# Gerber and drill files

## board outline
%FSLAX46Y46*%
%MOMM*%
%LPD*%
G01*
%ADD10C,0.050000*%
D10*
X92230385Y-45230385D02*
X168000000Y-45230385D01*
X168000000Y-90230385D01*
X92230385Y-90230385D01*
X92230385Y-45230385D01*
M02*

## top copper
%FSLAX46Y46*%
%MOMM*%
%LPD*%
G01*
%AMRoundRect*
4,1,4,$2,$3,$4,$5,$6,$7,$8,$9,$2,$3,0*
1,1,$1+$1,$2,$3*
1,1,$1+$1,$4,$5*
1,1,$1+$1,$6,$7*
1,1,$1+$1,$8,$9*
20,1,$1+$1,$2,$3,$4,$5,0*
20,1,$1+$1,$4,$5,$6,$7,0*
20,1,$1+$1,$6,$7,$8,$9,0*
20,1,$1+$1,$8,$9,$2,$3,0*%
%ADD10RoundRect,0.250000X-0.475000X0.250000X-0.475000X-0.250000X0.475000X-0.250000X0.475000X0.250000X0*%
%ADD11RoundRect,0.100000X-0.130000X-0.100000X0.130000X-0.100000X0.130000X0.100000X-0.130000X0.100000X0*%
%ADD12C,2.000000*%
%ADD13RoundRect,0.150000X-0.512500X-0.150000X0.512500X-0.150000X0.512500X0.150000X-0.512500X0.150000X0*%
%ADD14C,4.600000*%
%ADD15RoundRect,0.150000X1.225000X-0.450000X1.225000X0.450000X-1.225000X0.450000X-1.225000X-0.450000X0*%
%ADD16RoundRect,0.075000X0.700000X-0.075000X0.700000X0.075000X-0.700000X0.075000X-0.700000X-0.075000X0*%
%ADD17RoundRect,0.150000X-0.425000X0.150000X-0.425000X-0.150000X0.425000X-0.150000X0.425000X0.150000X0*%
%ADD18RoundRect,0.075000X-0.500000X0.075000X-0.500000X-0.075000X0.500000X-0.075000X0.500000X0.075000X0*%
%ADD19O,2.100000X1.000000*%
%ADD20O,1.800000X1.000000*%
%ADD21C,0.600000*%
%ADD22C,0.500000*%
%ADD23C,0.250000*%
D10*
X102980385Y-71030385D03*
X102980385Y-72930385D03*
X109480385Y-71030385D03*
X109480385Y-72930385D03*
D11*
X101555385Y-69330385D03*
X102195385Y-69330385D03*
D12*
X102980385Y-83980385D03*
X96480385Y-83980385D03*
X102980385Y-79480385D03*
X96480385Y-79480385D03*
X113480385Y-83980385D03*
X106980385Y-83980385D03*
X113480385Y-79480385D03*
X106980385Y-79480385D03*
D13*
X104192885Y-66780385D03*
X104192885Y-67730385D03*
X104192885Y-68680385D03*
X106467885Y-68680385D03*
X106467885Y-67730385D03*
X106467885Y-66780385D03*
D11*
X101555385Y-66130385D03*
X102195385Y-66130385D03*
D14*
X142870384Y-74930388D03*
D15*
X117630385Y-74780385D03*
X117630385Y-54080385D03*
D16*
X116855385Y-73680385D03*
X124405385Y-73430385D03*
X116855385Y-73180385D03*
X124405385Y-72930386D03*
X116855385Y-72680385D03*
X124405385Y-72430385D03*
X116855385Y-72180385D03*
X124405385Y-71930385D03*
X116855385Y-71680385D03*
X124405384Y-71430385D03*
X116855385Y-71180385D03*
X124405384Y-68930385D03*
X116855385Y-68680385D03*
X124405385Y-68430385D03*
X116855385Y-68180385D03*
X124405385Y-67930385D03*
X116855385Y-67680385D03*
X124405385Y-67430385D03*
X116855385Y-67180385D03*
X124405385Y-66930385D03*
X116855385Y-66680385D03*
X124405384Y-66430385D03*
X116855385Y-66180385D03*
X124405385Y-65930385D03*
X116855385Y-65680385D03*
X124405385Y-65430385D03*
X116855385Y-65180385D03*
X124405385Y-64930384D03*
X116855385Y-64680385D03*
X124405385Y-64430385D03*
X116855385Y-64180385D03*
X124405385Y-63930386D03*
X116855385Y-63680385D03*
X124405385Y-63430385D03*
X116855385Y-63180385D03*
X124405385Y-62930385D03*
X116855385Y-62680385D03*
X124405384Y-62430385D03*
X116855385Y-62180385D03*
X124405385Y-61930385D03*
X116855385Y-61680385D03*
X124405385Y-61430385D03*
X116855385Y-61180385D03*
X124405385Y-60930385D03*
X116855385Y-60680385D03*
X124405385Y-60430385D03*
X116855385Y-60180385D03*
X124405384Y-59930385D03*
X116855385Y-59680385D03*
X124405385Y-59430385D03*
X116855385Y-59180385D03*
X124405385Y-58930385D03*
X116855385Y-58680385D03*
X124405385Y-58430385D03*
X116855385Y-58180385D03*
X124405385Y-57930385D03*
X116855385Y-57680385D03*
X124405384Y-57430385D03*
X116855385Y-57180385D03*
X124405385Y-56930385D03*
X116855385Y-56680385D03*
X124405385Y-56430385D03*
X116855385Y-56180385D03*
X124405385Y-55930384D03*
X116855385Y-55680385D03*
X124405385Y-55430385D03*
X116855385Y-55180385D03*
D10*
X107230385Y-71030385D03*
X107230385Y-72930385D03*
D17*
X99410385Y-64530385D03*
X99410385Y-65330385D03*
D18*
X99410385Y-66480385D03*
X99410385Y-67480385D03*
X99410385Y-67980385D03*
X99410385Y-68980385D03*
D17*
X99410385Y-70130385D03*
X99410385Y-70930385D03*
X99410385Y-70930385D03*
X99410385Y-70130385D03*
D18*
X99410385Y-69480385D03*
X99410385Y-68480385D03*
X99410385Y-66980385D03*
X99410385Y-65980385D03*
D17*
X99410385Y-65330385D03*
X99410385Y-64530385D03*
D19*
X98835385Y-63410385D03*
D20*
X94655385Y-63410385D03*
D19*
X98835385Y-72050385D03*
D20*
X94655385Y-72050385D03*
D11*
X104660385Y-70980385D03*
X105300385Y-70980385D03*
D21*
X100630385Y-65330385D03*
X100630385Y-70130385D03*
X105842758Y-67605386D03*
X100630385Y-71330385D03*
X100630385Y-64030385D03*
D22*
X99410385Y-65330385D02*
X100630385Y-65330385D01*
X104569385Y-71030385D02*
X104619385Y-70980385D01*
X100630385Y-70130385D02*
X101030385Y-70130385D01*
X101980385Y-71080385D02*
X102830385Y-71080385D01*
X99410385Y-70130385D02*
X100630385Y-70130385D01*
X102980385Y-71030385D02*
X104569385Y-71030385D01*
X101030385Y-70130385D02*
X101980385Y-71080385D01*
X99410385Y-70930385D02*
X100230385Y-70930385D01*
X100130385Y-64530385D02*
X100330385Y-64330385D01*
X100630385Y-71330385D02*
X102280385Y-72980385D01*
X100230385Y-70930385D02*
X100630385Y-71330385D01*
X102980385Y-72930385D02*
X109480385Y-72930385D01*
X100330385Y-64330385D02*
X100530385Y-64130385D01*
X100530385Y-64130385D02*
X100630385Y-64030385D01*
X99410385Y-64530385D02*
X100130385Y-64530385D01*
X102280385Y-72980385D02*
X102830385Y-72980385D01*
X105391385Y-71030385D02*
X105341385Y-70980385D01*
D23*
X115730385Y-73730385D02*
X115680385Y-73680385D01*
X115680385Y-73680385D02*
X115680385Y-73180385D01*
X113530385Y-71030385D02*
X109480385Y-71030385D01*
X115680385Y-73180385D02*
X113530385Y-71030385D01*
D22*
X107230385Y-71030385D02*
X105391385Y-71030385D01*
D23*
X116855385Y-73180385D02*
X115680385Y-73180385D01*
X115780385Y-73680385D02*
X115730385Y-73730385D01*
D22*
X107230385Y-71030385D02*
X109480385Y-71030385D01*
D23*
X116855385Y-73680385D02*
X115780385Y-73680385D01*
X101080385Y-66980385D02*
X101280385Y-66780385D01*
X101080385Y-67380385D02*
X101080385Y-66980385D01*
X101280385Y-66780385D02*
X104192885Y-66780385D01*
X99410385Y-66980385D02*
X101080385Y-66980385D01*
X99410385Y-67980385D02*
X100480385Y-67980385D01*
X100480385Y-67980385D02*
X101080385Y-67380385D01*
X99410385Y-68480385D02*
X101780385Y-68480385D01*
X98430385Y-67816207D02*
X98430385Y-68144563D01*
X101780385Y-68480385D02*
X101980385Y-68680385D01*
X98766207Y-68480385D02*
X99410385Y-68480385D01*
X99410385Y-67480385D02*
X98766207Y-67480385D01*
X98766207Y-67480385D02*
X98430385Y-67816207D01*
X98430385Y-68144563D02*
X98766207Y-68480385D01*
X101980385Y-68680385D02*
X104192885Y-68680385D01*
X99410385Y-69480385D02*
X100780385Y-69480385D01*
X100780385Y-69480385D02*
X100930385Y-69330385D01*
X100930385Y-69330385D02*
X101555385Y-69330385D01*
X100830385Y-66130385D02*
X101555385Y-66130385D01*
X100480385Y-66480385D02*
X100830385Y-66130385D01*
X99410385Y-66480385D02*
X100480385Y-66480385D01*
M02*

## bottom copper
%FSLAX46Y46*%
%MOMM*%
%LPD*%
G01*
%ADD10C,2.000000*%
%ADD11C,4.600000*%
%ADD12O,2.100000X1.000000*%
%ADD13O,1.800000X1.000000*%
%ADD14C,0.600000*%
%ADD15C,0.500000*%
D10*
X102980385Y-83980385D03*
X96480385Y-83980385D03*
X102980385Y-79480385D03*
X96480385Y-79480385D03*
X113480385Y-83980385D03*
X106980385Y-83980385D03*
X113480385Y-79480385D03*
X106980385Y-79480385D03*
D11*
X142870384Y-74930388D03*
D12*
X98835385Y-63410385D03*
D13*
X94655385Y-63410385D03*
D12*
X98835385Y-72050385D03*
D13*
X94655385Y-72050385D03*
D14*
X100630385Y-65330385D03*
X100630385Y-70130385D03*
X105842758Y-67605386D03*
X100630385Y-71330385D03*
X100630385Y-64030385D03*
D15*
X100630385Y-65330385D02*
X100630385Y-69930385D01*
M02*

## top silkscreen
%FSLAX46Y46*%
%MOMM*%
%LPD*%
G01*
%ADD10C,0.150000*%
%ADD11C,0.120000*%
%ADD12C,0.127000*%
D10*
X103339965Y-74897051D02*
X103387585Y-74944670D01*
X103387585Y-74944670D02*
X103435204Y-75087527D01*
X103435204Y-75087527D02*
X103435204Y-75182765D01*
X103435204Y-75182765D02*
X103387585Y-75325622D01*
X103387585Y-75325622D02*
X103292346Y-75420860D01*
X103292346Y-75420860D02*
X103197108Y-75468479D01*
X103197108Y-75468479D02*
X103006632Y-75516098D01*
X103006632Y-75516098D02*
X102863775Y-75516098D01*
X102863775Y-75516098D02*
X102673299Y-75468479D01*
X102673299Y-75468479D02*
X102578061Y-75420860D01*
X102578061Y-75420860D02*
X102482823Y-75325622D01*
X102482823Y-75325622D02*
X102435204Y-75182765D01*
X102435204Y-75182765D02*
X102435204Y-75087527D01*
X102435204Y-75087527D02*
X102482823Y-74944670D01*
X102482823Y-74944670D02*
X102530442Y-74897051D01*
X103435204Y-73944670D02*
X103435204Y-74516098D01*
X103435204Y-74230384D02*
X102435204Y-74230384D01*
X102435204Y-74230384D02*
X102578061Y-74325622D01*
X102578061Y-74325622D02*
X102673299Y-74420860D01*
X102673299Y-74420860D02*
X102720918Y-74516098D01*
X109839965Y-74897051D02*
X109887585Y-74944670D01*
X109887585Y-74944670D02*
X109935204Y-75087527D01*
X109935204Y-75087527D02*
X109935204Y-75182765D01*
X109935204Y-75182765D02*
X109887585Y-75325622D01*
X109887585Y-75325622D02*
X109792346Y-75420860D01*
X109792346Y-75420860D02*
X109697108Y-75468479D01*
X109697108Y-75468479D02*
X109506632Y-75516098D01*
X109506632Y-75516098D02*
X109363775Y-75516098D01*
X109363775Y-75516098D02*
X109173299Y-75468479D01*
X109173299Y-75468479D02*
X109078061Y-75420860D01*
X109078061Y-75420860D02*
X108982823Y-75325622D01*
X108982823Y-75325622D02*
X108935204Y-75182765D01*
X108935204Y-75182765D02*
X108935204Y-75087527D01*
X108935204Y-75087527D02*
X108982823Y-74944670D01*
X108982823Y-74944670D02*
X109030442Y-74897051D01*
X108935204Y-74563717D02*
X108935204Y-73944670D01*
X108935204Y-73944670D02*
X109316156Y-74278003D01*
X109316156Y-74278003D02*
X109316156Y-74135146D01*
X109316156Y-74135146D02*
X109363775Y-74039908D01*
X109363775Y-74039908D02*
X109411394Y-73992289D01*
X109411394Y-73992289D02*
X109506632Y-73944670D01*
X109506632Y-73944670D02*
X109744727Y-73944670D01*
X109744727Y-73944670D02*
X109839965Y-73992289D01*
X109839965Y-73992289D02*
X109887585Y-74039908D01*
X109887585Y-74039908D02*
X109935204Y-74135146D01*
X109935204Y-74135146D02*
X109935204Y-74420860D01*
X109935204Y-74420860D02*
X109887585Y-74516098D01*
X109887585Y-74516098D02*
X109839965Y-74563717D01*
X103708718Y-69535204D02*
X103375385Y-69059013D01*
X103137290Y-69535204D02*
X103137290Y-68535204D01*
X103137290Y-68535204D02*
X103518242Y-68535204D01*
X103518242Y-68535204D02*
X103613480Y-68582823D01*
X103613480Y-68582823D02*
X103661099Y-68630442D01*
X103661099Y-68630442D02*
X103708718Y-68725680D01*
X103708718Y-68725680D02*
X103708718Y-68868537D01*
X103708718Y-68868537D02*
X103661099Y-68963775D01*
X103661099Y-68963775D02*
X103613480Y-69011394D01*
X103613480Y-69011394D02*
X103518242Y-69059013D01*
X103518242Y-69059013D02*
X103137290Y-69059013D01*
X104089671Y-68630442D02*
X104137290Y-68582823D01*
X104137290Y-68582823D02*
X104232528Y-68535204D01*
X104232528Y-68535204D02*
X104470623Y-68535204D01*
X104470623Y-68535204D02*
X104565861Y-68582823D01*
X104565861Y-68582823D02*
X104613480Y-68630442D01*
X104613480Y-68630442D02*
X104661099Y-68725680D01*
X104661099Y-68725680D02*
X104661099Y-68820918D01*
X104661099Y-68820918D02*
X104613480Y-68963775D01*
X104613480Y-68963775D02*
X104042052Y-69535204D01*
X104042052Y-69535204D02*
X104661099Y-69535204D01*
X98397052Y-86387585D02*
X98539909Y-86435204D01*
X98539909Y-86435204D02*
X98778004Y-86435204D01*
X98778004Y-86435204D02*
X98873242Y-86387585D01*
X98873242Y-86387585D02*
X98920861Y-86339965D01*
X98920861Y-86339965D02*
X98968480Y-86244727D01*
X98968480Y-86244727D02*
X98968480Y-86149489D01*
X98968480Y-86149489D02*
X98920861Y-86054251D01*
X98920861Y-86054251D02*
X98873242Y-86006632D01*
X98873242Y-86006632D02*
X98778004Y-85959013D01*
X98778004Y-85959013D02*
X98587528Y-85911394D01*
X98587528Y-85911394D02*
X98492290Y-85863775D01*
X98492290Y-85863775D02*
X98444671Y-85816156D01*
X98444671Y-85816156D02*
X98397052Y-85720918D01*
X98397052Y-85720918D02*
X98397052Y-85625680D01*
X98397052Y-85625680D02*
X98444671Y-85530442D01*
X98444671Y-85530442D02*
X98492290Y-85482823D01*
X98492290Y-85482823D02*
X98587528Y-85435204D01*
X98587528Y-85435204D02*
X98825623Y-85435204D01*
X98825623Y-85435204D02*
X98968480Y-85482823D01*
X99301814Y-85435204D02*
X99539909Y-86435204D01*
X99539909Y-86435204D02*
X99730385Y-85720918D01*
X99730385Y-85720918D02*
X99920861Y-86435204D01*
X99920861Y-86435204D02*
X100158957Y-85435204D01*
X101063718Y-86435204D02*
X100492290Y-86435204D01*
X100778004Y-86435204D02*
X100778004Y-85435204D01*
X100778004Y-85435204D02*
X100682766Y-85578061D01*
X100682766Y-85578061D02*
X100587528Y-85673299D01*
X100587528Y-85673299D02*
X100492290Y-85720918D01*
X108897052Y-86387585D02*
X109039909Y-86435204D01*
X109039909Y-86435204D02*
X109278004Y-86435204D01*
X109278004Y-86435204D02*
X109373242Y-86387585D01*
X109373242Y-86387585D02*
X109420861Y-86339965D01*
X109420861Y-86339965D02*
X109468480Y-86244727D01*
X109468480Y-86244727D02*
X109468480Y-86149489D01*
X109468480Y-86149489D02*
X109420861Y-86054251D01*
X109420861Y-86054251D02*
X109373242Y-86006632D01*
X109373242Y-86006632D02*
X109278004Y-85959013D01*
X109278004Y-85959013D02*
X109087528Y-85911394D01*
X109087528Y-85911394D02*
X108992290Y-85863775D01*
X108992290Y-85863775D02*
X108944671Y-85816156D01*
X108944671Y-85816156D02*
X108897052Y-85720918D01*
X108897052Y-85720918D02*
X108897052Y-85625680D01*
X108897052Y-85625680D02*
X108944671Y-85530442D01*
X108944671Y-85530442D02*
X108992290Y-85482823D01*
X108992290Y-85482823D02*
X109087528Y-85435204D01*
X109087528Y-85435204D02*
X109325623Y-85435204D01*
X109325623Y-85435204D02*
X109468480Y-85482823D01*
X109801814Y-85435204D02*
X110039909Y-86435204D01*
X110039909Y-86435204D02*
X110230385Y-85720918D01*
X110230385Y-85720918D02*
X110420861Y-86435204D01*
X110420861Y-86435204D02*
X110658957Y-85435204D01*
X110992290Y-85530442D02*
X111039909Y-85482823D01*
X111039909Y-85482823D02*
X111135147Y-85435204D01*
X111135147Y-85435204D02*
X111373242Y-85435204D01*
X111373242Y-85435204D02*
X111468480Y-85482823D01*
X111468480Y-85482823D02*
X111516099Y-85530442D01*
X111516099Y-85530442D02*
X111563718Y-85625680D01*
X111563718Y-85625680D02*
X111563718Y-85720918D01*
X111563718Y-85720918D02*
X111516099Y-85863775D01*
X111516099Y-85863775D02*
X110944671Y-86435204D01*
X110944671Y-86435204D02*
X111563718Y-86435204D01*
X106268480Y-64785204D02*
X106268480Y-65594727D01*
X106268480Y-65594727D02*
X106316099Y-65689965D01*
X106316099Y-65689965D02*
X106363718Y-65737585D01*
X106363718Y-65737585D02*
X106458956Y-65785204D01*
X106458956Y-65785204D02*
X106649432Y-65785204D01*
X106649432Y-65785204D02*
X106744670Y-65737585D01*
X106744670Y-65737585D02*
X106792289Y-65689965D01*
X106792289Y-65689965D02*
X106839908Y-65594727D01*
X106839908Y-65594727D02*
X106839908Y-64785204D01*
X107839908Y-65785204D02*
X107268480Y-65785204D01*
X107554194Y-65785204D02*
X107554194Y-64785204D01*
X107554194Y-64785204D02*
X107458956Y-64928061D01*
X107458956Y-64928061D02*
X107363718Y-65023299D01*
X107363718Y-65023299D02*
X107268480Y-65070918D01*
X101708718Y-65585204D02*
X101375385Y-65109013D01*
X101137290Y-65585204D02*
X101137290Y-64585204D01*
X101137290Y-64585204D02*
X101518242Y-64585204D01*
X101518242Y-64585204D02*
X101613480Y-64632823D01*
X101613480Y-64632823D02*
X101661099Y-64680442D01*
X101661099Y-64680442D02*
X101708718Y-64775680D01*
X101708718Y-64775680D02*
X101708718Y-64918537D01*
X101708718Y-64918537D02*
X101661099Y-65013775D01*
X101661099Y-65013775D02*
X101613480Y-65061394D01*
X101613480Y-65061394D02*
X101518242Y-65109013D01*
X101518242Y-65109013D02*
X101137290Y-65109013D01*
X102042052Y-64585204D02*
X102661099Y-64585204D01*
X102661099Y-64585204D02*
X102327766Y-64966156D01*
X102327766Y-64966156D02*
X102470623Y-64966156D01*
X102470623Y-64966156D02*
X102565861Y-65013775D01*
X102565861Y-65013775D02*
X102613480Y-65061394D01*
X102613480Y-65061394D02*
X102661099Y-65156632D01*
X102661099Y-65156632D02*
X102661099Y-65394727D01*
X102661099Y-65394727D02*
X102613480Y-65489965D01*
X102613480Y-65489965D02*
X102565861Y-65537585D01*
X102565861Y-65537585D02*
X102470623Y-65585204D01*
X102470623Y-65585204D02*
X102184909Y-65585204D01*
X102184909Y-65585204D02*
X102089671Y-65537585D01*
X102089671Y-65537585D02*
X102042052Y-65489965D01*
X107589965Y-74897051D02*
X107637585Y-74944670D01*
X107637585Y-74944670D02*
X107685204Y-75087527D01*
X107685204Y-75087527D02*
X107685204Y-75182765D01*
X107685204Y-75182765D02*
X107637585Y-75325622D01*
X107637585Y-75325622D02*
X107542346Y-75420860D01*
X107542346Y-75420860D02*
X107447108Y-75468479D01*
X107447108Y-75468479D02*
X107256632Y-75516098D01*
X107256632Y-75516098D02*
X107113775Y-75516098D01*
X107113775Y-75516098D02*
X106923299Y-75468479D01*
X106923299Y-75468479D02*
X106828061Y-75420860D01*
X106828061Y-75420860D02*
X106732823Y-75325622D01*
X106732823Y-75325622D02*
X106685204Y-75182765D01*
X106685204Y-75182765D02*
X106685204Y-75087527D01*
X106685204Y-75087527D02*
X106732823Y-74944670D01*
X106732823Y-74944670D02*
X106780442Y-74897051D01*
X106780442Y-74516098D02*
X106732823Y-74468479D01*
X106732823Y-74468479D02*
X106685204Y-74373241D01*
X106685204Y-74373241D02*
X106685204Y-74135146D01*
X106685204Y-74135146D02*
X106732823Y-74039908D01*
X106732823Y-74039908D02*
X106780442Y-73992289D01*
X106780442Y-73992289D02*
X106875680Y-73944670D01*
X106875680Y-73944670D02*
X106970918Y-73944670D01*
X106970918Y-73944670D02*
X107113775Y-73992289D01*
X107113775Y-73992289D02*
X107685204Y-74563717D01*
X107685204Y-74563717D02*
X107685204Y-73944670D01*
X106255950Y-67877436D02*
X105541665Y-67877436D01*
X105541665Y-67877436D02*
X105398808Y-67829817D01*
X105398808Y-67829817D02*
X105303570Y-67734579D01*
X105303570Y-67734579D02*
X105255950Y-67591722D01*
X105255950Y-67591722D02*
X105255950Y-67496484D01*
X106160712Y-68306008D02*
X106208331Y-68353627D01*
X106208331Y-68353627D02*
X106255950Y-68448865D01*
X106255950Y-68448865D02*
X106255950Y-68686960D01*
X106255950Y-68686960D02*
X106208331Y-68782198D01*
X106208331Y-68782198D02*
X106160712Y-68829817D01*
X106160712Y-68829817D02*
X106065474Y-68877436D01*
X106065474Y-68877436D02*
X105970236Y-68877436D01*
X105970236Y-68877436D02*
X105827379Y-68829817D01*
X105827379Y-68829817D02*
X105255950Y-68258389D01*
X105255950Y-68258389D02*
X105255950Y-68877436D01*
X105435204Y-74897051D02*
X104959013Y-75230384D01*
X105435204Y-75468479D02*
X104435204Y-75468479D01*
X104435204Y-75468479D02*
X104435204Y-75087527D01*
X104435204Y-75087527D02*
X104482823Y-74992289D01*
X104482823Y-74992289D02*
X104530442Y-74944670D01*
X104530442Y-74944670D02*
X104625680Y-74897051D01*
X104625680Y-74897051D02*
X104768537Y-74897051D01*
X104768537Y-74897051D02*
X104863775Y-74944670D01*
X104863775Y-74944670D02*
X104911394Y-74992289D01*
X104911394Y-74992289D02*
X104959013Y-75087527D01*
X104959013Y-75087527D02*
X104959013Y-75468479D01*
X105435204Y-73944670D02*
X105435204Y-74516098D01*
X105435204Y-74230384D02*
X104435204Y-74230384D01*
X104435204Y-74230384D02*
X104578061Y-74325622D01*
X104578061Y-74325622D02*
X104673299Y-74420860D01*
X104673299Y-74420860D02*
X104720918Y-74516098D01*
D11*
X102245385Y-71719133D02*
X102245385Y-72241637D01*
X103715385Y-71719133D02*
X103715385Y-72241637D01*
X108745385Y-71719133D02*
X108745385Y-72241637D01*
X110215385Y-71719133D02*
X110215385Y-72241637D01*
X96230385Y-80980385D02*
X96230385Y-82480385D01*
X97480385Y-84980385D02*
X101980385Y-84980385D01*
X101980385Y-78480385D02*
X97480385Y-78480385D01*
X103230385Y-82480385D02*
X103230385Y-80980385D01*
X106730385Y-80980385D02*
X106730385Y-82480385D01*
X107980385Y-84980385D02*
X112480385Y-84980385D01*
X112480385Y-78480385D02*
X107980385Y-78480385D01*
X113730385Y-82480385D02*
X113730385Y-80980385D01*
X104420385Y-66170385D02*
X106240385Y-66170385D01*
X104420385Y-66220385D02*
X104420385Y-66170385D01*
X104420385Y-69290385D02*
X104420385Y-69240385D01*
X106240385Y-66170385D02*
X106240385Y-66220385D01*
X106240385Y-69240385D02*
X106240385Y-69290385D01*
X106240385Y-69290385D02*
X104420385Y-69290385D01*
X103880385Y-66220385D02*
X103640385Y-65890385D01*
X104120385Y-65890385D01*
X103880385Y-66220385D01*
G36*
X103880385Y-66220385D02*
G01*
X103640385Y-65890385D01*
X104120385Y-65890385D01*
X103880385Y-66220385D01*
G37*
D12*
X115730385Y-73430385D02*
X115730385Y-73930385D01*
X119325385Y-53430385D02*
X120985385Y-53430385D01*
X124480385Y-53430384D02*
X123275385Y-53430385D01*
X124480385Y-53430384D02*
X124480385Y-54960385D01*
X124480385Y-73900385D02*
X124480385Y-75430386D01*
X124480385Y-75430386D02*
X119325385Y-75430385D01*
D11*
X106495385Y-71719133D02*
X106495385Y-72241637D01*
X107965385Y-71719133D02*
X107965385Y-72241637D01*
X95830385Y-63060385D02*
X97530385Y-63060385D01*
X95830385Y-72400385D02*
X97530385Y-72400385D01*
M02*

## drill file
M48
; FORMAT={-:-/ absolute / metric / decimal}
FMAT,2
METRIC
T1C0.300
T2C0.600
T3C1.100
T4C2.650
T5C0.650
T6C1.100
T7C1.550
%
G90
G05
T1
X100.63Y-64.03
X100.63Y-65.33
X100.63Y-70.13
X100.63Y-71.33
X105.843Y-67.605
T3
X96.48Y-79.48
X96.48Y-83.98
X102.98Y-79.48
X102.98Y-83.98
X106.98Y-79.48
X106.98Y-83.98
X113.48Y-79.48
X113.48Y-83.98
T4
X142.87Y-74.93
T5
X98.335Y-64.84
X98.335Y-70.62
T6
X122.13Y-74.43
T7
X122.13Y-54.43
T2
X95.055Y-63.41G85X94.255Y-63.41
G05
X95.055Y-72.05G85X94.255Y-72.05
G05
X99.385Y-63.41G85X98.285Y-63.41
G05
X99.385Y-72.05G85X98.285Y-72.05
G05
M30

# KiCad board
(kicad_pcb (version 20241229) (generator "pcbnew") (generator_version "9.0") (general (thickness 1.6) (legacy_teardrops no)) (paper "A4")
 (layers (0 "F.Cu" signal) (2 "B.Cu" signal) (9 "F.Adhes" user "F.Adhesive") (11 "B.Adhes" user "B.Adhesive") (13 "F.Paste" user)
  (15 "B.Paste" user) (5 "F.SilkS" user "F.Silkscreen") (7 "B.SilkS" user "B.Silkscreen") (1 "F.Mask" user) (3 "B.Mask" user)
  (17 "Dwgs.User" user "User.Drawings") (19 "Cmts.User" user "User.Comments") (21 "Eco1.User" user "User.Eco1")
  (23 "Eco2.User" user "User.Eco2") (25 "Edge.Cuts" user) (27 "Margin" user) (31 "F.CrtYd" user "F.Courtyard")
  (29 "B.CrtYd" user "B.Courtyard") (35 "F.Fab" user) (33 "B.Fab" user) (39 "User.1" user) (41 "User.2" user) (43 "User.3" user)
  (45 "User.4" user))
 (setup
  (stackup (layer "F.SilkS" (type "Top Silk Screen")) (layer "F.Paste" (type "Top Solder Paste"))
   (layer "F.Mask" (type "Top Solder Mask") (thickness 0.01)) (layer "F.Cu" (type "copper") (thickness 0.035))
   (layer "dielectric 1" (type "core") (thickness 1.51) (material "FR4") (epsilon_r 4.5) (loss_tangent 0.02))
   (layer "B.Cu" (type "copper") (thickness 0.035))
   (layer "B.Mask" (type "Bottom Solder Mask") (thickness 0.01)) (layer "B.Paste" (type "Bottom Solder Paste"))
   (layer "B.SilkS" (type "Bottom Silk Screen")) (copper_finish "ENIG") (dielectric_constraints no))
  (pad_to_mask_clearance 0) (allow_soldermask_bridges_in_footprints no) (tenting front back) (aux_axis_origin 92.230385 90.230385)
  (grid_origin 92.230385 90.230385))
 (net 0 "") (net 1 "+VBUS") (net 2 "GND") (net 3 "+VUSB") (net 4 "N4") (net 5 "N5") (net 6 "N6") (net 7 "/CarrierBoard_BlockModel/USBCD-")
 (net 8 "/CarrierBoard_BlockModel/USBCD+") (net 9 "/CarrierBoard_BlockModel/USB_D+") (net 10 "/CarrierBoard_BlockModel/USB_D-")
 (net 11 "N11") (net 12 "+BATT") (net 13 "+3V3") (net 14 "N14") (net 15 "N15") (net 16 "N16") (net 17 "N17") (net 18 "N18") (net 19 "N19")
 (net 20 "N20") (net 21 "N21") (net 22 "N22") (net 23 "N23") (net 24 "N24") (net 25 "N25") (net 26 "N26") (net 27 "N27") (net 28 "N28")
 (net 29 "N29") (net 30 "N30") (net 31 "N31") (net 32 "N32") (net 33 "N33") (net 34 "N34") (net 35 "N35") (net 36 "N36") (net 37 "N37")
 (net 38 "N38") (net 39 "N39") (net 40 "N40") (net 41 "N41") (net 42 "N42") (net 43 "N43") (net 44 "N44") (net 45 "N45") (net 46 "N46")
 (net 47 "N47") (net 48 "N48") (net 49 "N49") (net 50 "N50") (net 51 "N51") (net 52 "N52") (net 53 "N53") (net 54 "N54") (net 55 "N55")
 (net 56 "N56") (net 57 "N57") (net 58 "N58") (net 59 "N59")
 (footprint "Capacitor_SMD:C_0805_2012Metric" (layer "F.Cu") (at 102.980385 71.980385 -90)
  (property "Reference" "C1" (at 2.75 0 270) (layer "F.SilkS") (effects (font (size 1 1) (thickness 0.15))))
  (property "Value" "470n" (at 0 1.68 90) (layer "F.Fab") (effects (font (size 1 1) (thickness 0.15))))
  (fp_line (start -0.261252 0.735) (end 0.261252 0.735) (stroke (width 0.12) (type solid)) (layer "F.SilkS"))
  (fp_line (start -0.261252 -0.735) (end 0.261252 -0.735) (stroke (width 0.12) (type solid)) (layer "F.SilkS"))
  (pad "1" smd roundrect (at -0.95 0 270) (size 1 1.45) (layers "F.Cu" "F.Mask" "F.Paste") (roundrect_rratio 0.25) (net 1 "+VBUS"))
  (pad "2" smd roundrect (at 0.95 0 270) (size 1 1.45) (layers "F.Cu" "F.Mask" "F.Paste") (roundrect_rratio 0.25) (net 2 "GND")))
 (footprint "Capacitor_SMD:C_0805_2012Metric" (layer "F.Cu") (at 109.480385 71.980385 -90)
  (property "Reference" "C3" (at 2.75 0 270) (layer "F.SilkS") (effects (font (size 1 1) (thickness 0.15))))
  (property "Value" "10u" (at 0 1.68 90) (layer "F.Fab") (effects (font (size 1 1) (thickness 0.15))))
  (fp_line (start -0.261252 0.735) (end 0.261252 0.735) (stroke (width 0.12) (type solid)) (layer "F.SilkS"))
  (fp_line (start -0.261252 -0.735) (end 0.261252 -0.735) (stroke (width 0.12) (type solid)) (layer "F.SilkS"))
  (pad "1" smd roundrect (at -0.95 0 270) (size 1 1.45) (layers "F.Cu" "F.Mask" "F.Paste") (roundrect_rratio 0.25) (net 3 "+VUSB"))
  (pad "2" smd roundrect (at 0.95 0 270) (size 1 1.45) (layers "F.Cu" "F.Mask" "F.Paste") (roundrect_rratio 0.25) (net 2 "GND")))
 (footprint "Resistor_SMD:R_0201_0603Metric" (layer "F.Cu") (at 101.875385 69.330385)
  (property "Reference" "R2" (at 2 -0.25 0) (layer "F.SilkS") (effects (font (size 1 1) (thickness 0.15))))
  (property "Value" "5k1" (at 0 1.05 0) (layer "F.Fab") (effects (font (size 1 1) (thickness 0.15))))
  (pad "" smd roundrect (at -0.345 0) (size 0.318 0.36) (layers "F.Paste") (roundrect_rratio 0.25))
  (pad "" smd roundrect (at 0.345 0) (size 0.318 0.36) (layers "F.Paste") (roundrect_rratio 0.25))
  (pad "1" smd roundrect (at -0.32 0) (size 0.46 0.4) (layers "F.Cu" "F.Mask") (roundrect_rratio 0.25) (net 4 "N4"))
  (pad "2" smd roundrect (at 0.32 0) (size 0.46 0.4) (layers "F.Cu" "F.Mask") (roundrect_rratio 0.25) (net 2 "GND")))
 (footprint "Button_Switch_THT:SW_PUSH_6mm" (layer "F.Cu") (at 102.980385 83.980385 180)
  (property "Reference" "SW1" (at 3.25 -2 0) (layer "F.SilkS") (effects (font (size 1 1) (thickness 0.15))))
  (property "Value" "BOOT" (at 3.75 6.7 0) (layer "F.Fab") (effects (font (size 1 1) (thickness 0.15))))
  (fp_line (start 6.75 3) (end 6.75 1.5) (stroke (width 0.12) (type solid)) (layer "F.SilkS"))
  (fp_line (start 5.5 -1) (end 1 -1) (stroke (width 0.12) (type solid)) (layer "F.SilkS"))
  (fp_line (start 1 5.5) (end 5.5 5.5) (stroke (width 0.12) (type solid)) (layer "F.SilkS"))
  (fp_line (start -0.25 1.5) (end -0.25 3) (stroke (width 0.12) (type solid)) (layer "F.SilkS"))
  (pad "1" thru_hole circle (at 0 0 270) (size 2 2) (drill 1.1) (layers "*.Cu" "*.Mask") (remove_unused_layers no) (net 2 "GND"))
  (pad "1" thru_hole circle (at 6.5 0 270) (size 2 2) (drill 1.1) (layers "*.Cu" "*.Mask") (remove_unused_layers no) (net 2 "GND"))
  (pad "2" thru_hole circle (at 0 4.5 270) (size 2 2) (drill 1.1) (layers "*.Cu" "*.Mask") (remove_unused_layers no) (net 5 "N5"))
  (pad "2" thru_hole circle (at 6.5 4.5 270) (size 2 2) (drill 1.1) (layers "*.Cu" "*.Mask") (remove_unused_layers no) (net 5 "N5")))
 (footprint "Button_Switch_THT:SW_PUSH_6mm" (layer "F.Cu") (at 113.480385 83.980385 180)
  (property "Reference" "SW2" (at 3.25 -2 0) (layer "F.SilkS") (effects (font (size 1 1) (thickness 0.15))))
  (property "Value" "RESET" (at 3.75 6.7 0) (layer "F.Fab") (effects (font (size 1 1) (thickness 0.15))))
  (fp_line (start 6.75 3) (end 6.75 1.5) (stroke (width 0.12) (type solid)) (layer "F.SilkS"))
  (fp_line (start 5.5 -1) (end 1 -1) (stroke (width 0.12) (type solid)) (layer "F.SilkS"))
  (fp_line (start 1 5.5) (end 5.5 5.5) (stroke (width 0.12) (type solid)) (layer "F.SilkS"))
  (fp_line (start -0.25 1.5) (end -0.25 3) (stroke (width 0.12) (type solid)) (layer "F.SilkS"))
  (pad "1" thru_hole circle (at 0 0 270) (size 2 2) (drill 1.1) (layers "*.Cu" "*.Mask") (remove_unused_layers no) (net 2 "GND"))
  (pad "1" thru_hole circle (at 6.5 0 270) (size 2 2) (drill 1.1) (layers "*.Cu" "*.Mask") (remove_unused_layers no) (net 2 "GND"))
  (pad "2" thru_hole circle (at 0 4.5 270) (size 2 2) (drill 1.1) (layers "*.Cu" "*.Mask") (remove_unused_layers no) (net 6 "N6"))
  (pad "2" thru_hole circle (at 6.5 4.5 270) (size 2 2) (drill 1.1) (layers "*.Cu" "*.Mask") (remove_unused_layers no) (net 6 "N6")))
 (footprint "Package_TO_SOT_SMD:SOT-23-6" (layer "F.Cu") (at 105.330385 67.730385)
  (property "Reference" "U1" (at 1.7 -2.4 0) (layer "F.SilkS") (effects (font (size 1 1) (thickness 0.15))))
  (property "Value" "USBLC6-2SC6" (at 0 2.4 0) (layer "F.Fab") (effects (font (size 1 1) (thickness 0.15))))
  (fp_line (start -0.91 -1.56) (end 0.91 -1.56) (stroke (width 0.12) (type solid)) (layer "F.SilkS"))
  (fp_line (start -0.91 -1.51) (end -0.91 -1.56) (stroke (width 0.12) (type solid)) (layer "F.SilkS"))
  (fp_line (start -0.91 1.56) (end -0.91 1.51) (stroke (width 0.12) (type solid)) (layer "F.SilkS"))
  (fp_line (start 0.91 -1.56) (end 0.91 -1.51) (stroke (width 0.12) (type solid)) (layer "F.SilkS"))
  (fp_line (start 0.91 1.51) (end 0.91 1.56) (stroke (width 0.12) (type solid)) (layer "F.SilkS"))
  (fp_line (start 0.91 1.56) (end -0.91 1.56) (stroke (width 0.12) (type solid)) (layer "F.SilkS"))
  (fp_poly (pts (xy -1.45 -1.51) (xy -1.69 -1.84) (xy -1.21 -1.84)) (stroke (width 0.12) (type solid)) (fill yes) (layer "F.SilkS"))
  (pad "1" smd roundrect (at -1.1375 -0.95) (size 1.325 0.6) (layers "F.Cu" "F.Mask" "F.Paste") (roundrect_rratio 0.25)
   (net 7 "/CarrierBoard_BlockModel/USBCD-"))
  (pad "2" smd roundrect (at -1.1375 0) (size 1.325 0.6) (layers "F.Cu" "F.Mask" "F.Paste") (roundrect_rratio 0.25) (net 2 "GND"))
  (pad "3" smd roundrect (at -1.1375 0.95) (size 1.325 0.6) (layers "F.Cu" "F.Mask" "F.Paste") (roundrect_rratio 0.25)
   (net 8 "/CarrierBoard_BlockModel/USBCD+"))
  (pad "4" smd roundrect (at 1.1375 0.95) (size 1.325 0.6) (layers "F.Cu" "F.Mask" "F.Paste") (roundrect_rratio 0.25)
   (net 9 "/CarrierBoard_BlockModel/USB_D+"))
  (pad "5" smd roundrect (at 1.1375 0) (size 1.325 0.6) (layers "F.Cu" "F.Mask" "F.Paste") (roundrect_rratio 0.25) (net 1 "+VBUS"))
  (pad "6" smd roundrect (at 1.1375 -0.95) (size 1.325 0.6) (layers "F.Cu" "F.Mask" "F.Paste") (roundrect_rratio 0.25)
   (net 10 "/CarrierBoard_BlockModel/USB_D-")))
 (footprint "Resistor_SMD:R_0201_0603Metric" (layer "F.Cu") (at 101.875385 66.130385)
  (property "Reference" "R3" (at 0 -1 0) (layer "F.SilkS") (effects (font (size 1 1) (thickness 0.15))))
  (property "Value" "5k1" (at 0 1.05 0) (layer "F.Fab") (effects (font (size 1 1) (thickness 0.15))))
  (pad "" smd roundrect (at -0.345 0) (size 0.318 0.36) (layers "F.Paste") (roundrect_rratio 0.25))
  (pad "" smd roundrect (at 0.345 0) (size 0.318 0.36) (layers "F.Paste") (roundrect_rratio 0.25))
  (pad "1" smd roundrect (at -0.32 0) (size 0.46 0.4) (layers "F.Cu" "F.Mask") (roundrect_rratio 0.25) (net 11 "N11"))
  (pad "2" smd roundrect (at 0.32 0) (size 0.46 0.4) (layers "F.Cu" "F.Mask") (roundrect_rratio 0.25) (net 2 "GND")))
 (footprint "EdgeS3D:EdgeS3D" (layer "F.Cu") (at 122.130385 64.430385 90)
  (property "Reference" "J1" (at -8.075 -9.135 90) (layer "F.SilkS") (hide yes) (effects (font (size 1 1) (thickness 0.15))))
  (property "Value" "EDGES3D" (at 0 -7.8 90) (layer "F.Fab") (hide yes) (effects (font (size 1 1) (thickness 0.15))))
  (fp_line (start -9 -6.4) (end -9.5 -6.4) (stroke (width 0.127) (type solid)) (layer "F.SilkS"))
  (fp_line (start 11 -2.805) (end 11 -1.145) (stroke (width 0.127) (type solid)) (layer "F.SilkS"))
  (fp_line (start 11.000001 2.35) (end 11 1.145) (stroke (width 0.127) (type solid)) (layer "F.SilkS"))
  (fp_line (start 11.000001 2.35) (end 9.47 2.35) (stroke (width 0.127) (type solid)) (layer "F.SilkS"))
  (fp_line (start -9.47 2.35) (end -11.000001 2.35) (stroke (width 0.127) (type solid)) (layer "F.SilkS"))
  (fp_line (start -11.000001 2.35) (end -11 -2.805) (stroke (width 0.127) (type solid)) (layer "F.SilkS"))
  (pad "" thru_hole circle (at -10.500003 20.739999 90) (size 4.6 4.6) (drill 2.65) (layers "*.Cu" "F.Mask") (remove_unused_layers no))
  (pad "" smd roundrect (at -10.35 -4.5 90) (size 1.2 2.75) (layers "F.Cu" "F.Mask" "F.Paste") (roundrect_rratio 0.125)
   (solder_mask_margin 0.01))
  (pad "" np_thru_hole circle (at -10 0 90) (size 1.1 1.1) (drill 1.1) (layers "*.Cu" "*.Mask"))
  (pad "" np_thru_hole circle (at 10 0 90) (size 1.55 1.55) (drill 1.55) (layers "*.Cu" "*.Mask"))
  (pad "" smd roundrect (at 10.35 -4.5 90) (size 1.2 2.75) (layers "F.Cu" "F.Mask" "F.Paste") (roundrect_rratio 0.125)
   (solder_mask_margin 0.01))
  (pad "1" smd roundrect (at -9.25 -5.275 90) (size 0.3 1.55) (layers "F.Cu" "F.Mask" "F.Paste") (roundrect_rratio 0.25) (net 3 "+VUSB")
   (solder_mask_margin 0.01))
  (pad "2" smd roundrect (at -9 2.275 90) (size 0.3 1.55) (layers "F.Cu" "F.Mask" "F.Paste") (roundrect_rratio 0.25) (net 2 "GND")
   (solder_mask_margin 0.01))
  (pad "3" smd roundrect (at -8.75 -5.275 90) (size 0.3 1.55) (layers "F.Cu" "F.Mask" "F.Paste") (roundrect_rratio 0.25) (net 3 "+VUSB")
   (solder_mask_margin 0.01))
  (pad "4" smd roundrect (at -8.500001 2.275 90) (size 0.3 1.55) (layers "F.Cu" "F.Mask" "F.Paste") (roundrect_rratio 0.25) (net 2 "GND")
   (solder_mask_margin 0.01))
  (pad "5" smd roundrect (at -8.25 -5.275 90) (size 0.3 1.55) (layers "F.Cu" "F.Mask" "F.Paste") (roundrect_rratio 0.25) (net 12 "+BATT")
   (solder_mask_margin 0.01))
  (pad "6" smd roundrect (at -8 2.275 90) (size 0.3 1.55) (layers "F.Cu" "F.Mask" "F.Paste") (roundrect_rratio 0.25) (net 2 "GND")
   (solder_mask_margin 0.01))
  (pad "7" smd roundrect (at -7.75 -5.275 90) (size 0.3 1.55) (layers "F.Cu" "F.Mask" "F.Paste") (roundrect_rratio 0.25) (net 12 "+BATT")
   (solder_mask_margin 0.01))
  (pad "8" smd roundrect (at -7.5 2.275 90) (size 0.3 1.55) (layers "F.Cu" "F.Mask" "F.Paste") (roundrect_rratio 0.25) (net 2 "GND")
   (solder_mask_margin 0.01))
  (pad "9" smd roundrect (at -7.25 -5.275 90) (size 0.3 1.55) (layers "F.Cu" "F.Mask" "F.Paste") (roundrect_rratio 0.25) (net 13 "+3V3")
   (solder_mask_margin 0.01))
  (pad "10" smd roundrect (at -7 2.274999 90) (size 0.3 1.55) (layers "F.Cu" "F.Mask" "F.Paste") (roundrect_rratio 0.25) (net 2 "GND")
   (solder_mask_margin 0.01))
  (pad "11" smd roundrect (at -6.75 -5.275 90) (size 0.3 1.55) (layers "F.Cu" "F.Mask" "F.Paste") (roundrect_rratio 0.25) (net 13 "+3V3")
   (solder_mask_margin 0.01))
  (pad "20" smd roundrect (at -4.5 2.274999 90) (size 0.3 1.55) (layers "F.Cu" "F.Mask" "F.Paste") (roundrect_rratio 0.25) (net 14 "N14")
   (solder_mask_margin 0.01))
  (pad "21" smd roundrect (at -4.25 -5.275 90) (size 0.3 1.55) (layers "F.Cu" "F.Mask" "F.Paste") (roundrect_rratio 0.25) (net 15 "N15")
   (solder_mask_margin 0.01))
  (pad "22" smd roundrect (at -4 2.275 90) (size 0.3 1.55) (layers "F.Cu" "F.Mask" "F.Paste") (roundrect_rratio 0.25) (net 5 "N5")
   (solder_mask_margin 0.01))
  (pad "23" smd roundrect (at -3.75 -5.275 90) (size 0.3 1.55) (layers "F.Cu" "F.Mask" "F.Paste") (roundrect_rratio 0.25) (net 6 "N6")
   (solder_mask_margin 0.01))
  (pad "24" smd roundrect (at -3.5 2.275 90) (size 0.3 1.55) (layers "F.Cu" "F.Mask" "F.Paste") (roundrect_rratio 0.25) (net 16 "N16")
   (solder_mask_margin 0.01))
  (pad "25" smd roundrect (at -3.25 -5.275 90) (size 0.3 1.55) (layers "F.Cu" "F.Mask" "F.Paste") (roundrect_rratio 0.25) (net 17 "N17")
   (solder_mask_margin 0.01))
  (pad "26" smd roundrect (at -3 2.275 90) (size 0.3 1.55) (layers "F.Cu" "F.Mask" "F.Paste") (roundrect_rratio 0.25) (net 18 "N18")
   (solder_mask_margin 0.01))
  (pad "27" smd roundrect (at -2.75 -5.275 90) (size 0.3 1.55) (layers "F.Cu" "F.Mask" "F.Paste") (roundrect_rratio 0.25) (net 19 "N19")
   (solder_mask_margin 0.01))
  (pad "28" smd roundrect (at -2.5 2.275 90) (size 0.3 1.55) (layers "F.Cu" "F.Mask" "F.Paste") (roundrect_rratio 0.25) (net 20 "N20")
   (solder_mask_margin 0.01))
  (pad "29" smd roundrect (at -2.25 -5.275 90) (size 0.3 1.55) (layers "F.Cu" "F.Mask" "F.Paste") (roundrect_rratio 0.25) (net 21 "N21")
   (solder_mask_margin 0.01))
  (pad "30" smd roundrect (at -2 2.274999 90) (size 0.3 1.55) (layers "F.Cu" "F.Mask" "F.Paste") (roundrect_rratio 0.25) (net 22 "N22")
   (solder_mask_margin 0.01))
  (pad "31" smd roundrect (at -1.75 -5.275 90) (size 0.3 1.55) (layers "F.Cu" "F.Mask" "F.Paste") (roundrect_rratio 0.25) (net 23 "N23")
   (solder_mask_margin 0.01))
  (pad "32" smd roundrect (at -1.5 2.275 90) (size 0.3 1.55) (layers "F.Cu" "F.Mask" "F.Paste") (roundrect_rratio 0.25) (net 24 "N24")
   (solder_mask_margin 0.01))
  (pad "33" smd roundrect (at -1.25 -5.275 90) (size 0.3 1.55) (layers "F.Cu" "F.Mask" "F.Paste") (roundrect_rratio 0.25) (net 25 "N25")
   (solder_mask_margin 0.01))
  (pad "34" smd roundrect (at -1 2.275 90) (size 0.3 1.55) (layers "F.Cu" "F.Mask" "F.Paste") (roundrect_rratio 0.25) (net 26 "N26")
   (solder_mask_margin 0.01))
  (pad "35" smd roundrect (at -0.75 -5.275 90) (size 0.3 1.55) (layers "F.Cu" "F.Mask" "F.Paste") (roundrect_rratio 0.25) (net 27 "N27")
   (solder_mask_margin 0.01))
  (pad "36" smd roundrect (at -0.499999 2.275 90) (size 0.3 1.55) (layers "F.Cu" "F.Mask" "F.Paste") (roundrect_rratio 0.25) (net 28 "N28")
   (solder_mask_margin 0.01))
  (pad "37" smd roundrect (at -0.25 -5.275 90) (size 0.3 1.55) (layers "F.Cu" "F.Mask" "F.Paste") (roundrect_rratio 0.25) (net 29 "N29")
   (solder_mask_margin 0.01))
  (pad "38" smd roundrect (at 0 2.275 90) (size 0.3 1.55) (layers "F.Cu" "F.Mask" "F.Paste") (roundrect_rratio 0.25) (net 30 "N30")
   (solder_mask_margin 0.01))
  (pad "39" smd roundrect (at 0.25 -5.275 90) (size 0.3 1.55) (layers "F.Cu" "F.Mask" "F.Paste") (roundrect_rratio 0.25) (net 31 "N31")
   (solder_mask_margin 0.01))
  (pad "40" smd roundrect (at 0.499999 2.275 90) (size 0.3 1.55) (layers "F.Cu" "F.Mask" "F.Paste") (roundrect_rratio 0.25) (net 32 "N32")
   (solder_mask_margin 0.01))
  (pad "41" smd roundrect (at 0.75 -5.275 90) (size 0.3 1.55) (layers "F.Cu" "F.Mask" "F.Paste") (roundrect_rratio 0.25) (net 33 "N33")
   (solder_mask_margin 0.01))
  (pad "42" smd roundrect (at 1 2.275 90) (size 0.3 1.55) (layers "F.Cu" "F.Mask" "F.Paste") (roundrect_rratio 0.25) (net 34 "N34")
   (solder_mask_margin 0.01))
  (pad "43" smd roundrect (at 1.25 -5.275 90) (size 0.3 1.55) (layers "F.Cu" "F.Mask" "F.Paste") (roundrect_rratio 0.25) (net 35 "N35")
   (solder_mask_margin 0.01))
  (pad "44" smd roundrect (at 1.5 2.275 90) (size 0.3 1.55) (layers "F.Cu" "F.Mask" "F.Paste") (roundrect_rratio 0.25) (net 2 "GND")
   (solder_mask_margin 0.01))
  (pad "45" smd roundrect (at 1.75 -5.275 90) (size 0.3 1.55) (layers "F.Cu" "F.Mask" "F.Paste") (roundrect_rratio 0.25) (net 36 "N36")
   (solder_mask_margin 0.01))
  (pad "46" smd roundrect (at 2 2.274999 90) (size 0.3 1.55) (layers "F.Cu" "F.Mask" "F.Paste") (roundrect_rratio 0.25)
   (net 10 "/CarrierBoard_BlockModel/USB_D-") (solder_mask_margin 0.01))
  (pad "47" smd roundrect (at 2.25 -5.275 90) (size 0.3 1.55) (layers "F.Cu" "F.Mask" "F.Paste") (roundrect_rratio 0.25) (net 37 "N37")
   (solder_mask_margin 0.01))
  (pad "48" smd roundrect (at 2.5 2.275 90) (size 0.3 1.55) (layers "F.Cu" "F.Mask" "F.Paste") (roundrect_rratio 0.25)
   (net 9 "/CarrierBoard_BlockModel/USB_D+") (solder_mask_margin 0.01))
  (pad "49" smd roundrect (at 2.75 -5.275 90) (size 0.3 1.55) (layers "F.Cu" "F.Mask" "F.Paste") (roundrect_rratio 0.25) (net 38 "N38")
   (solder_mask_margin 0.01))
  (pad "50" smd roundrect (at 3 2.275 90) (size 0.3 1.55) (layers "F.Cu" "F.Mask" "F.Paste") (roundrect_rratio 0.25) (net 2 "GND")
   (solder_mask_margin 0.01))
  (pad "51" smd roundrect (at 3.25 -5.275 90) (size 0.3 1.55) (layers "F.Cu" "F.Mask" "F.Paste") (roundrect_rratio 0.25) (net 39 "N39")
   (solder_mask_margin 0.01))
  (pad "52" smd roundrect (at 3.5 2.275 90) (size 0.3 1.55) (layers "F.Cu" "F.Mask" "F.Paste") (roundrect_rratio 0.25) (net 2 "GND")
   (solder_mask_margin 0.01))
  (pad "53" smd roundrect (at 3.75 -5.275 90) (size 0.3 1.55) (layers "F.Cu" "F.Mask" "F.Paste") (roundrect_rratio 0.25) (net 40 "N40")
   (solder_mask_margin 0.01))
  (pad "54" smd roundrect (at 4 2.275 90) (size 0.3 1.55) (layers "F.Cu" "F.Mask" "F.Paste") (roundrect_rratio 0.25) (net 2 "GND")
   (solder_mask_margin 0.01))
  (pad "55" smd roundrect (at 4.25 -5.275 90) (size 0.3 1.55) (layers "F.Cu" "F.Mask" "F.Paste") (roundrect_rratio 0.25) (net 2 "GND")
   (solder_mask_margin 0.01))
  (pad "56" smd roundrect (at 4.5 2.274999 90) (size 0.3 1.55) (layers "F.Cu" "F.Mask" "F.Paste") (roundrect_rratio 0.25) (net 2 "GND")
   (solder_mask_margin 0.01))
  (pad "57" smd roundrect (at 4.75 -5.275 90) (size 0.3 1.55) (layers "F.Cu" "F.Mask" "F.Paste") (roundrect_rratio 0.25) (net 2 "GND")
   (solder_mask_margin 0.01))
  (pad "58" smd roundrect (at 5 2.275 90) (size 0.3 1.55) (layers "F.Cu" "F.Mask" "F.Paste") (roundrect_rratio 0.25) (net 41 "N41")
   (solder_mask_margin 0.01))
  (pad "59" smd roundrect (at 5.25 -5.275 90) (size 0.3 1.55) (layers "F.Cu" "F.Mask" "F.Paste") (roundrect_rratio 0.25) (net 2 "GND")
   (solder_mask_margin 0.01))
  (pad "60" smd roundrect (at 5.5 2.275 90) (size 0.3 1.55) (layers "F.Cu" "F.Mask" "F.Paste") (roundrect_rratio 0.25) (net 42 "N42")
   (solder_mask_margin 0.01))
  (pad "61" smd roundrect (at 5.75 -5.275 90) (size 0.3 1.55) (layers "F.Cu" "F.Mask" "F.Paste") (roundrect_rratio 0.25) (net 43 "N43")
   (solder_mask_margin 0.01))
  (pad "62" smd roundrect (at 6 2.275 90) (size 0.3 1.55) (layers "F.Cu" "F.Mask" "F.Paste") (roundrect_rratio 0.25) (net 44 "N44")
   (solder_mask_margin 0.01))
  (pad "63" smd roundrect (at 6.25 -5.275 90) (size 0.3 1.55) (layers "F.Cu" "F.Mask" "F.Paste") (roundrect_rratio 0.25) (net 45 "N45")
   (solder_mask_margin 0.01))
  (pad "64" smd roundrect (at 6.5 2.275 90) (size 0.3 1.55) (layers "F.Cu" "F.Mask" "F.Paste") (roundrect_rratio 0.25) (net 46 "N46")
   (solder_mask_margin 0.01))
  (pad "65" smd roundrect (at 6.75 -5.275 90) (size 0.3 1.55) (layers "F.Cu" "F.Mask" "F.Paste") (roundrect_rratio 0.25) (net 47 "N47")
   (solder_mask_margin 0.01))
  (pad "66" smd roundrect (at 7 2.274999 90) (size 0.3 1.55) (layers "F.Cu" "F.Mask" "F.Paste") (roundrect_rratio 0.25) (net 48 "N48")
   (solder_mask_margin 0.01))
  (pad "67" smd roundrect (at 7.25 -5.275 90) (size 0.3 1.55) (layers "F.Cu" "F.Mask" "F.Paste") (roundrect_rratio 0.25) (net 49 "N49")
   (solder_mask_margin 0.01))
  (pad "68" smd roundrect (at 7.5 2.275 90) (size 0.3 1.55) (layers "F.Cu" "F.Mask" "F.Paste") (roundrect_rratio 0.25) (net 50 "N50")
   (solder_mask_margin 0.01))
  (pad "69" smd roundrect (at 7.75 -5.275 90) (size 0.3 1.55) (layers "F.Cu" "F.Mask" "F.Paste") (roundrect_rratio 0.25) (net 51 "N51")
   (solder_mask_margin 0.01))
  (pad "70" smd roundrect (at 8 2.275 90) (size 0.3 1.55) (layers "F.Cu" "F.Mask" "F.Paste") (roundrect_rratio 0.25) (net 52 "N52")
   (solder_mask_margin 0.01))
  (pad "71" smd roundrect (at 8.25 -5.275 90) (size 0.3 1.55) (layers "F.Cu" "F.Mask" "F.Paste") (roundrect_rratio 0.25) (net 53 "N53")
   (solder_mask_margin 0.01))
  (pad "72" smd roundrect (at 8.500001 2.275 90) (size 0.3 1.55) (layers "F.Cu" "F.Mask" "F.Paste") (roundrect_rratio 0.25) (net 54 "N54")
   (solder_mask_margin 0.01))
  (pad "73" smd roundrect (at 8.75 -5.275 90) (size 0.3 1.55) (layers "F.Cu" "F.Mask" "F.Paste") (roundrect_rratio 0.25) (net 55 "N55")
   (solder_mask_margin 0.01))
  (pad "74" smd roundrect (at 9 2.275 90) (size 0.3 1.55) (layers "F.Cu" "F.Mask" "F.Paste") (roundrect_rratio 0.25) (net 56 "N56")
   (solder_mask_margin 0.01))
  (pad "75" smd roundrect (at 9.25 -5.275 90) (size 0.3 1.55) (layers "F.Cu" "F.Mask" "F.Paste") (roundrect_rratio 0.25) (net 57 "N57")
   (solder_mask_margin 0.01)))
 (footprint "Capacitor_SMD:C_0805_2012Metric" (layer "F.Cu") (at 107.230385 71.980385 -90)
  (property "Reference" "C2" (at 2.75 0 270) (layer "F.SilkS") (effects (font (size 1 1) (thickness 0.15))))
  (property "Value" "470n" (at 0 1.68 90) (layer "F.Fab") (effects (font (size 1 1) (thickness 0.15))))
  (fp_line (start -0.261252 0.735) (end 0.261252 0.735) (stroke (width 0.12) (type solid)) (layer "F.SilkS"))
  (fp_line (start -0.261252 -0.735) (end 0.261252 -0.735) (stroke (width 0.12) (type solid)) (layer "F.SilkS"))
  (pad "1" smd roundrect (at -0.95 0 270) (size 1 1.45) (layers "F.Cu" "F.Mask" "F.Paste") (roundrect_rratio 0.25) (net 3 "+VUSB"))
  (pad "2" smd roundrect (at 0.95 0 270) (size 1 1.45) (layers "F.Cu" "F.Mask" "F.Paste") (roundrect_rratio 0.25) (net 2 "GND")))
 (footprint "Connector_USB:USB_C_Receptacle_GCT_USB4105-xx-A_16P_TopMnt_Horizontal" (layer "F.Cu") (at 95.730385 67.730385 -90)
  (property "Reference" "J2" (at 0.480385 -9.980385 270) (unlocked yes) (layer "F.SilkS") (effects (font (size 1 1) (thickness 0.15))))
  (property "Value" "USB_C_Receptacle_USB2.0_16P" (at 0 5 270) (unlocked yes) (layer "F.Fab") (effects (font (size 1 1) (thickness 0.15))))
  (fp_line (start -4.67 -0.1) (end -4.67 -1.8) (stroke (width 0.12) (type solid)) (layer "F.SilkS"))
  (fp_line (start 4.67 -0.1) (end 4.67 -1.8) (stroke (width 0.12) (type solid)) (layer "F.SilkS"))
  (pad "" np_thru_hole circle (at -2.89 -2.605 270) (size 0.65 0.65) (drill 0.65) (layers "*.Cu" "*.Mask"))
  (pad "" np_thru_hole circle (at 2.89 -2.605 270) (size 0.65 0.65) (drill 0.65) (layers "*.Cu" "*.Mask"))
  (pad "A1" smd roundrect (at -3.2 -3.68 270) (size 0.6 1.15) (layers "F.Cu" "F.Mask" "F.Paste") (roundrect_rratio 0.25) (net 2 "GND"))
  (pad "A4" smd roundrect (at -2.4 -3.68 270) (size 0.6 1.15) (layers "F.Cu" "F.Mask" "F.Paste") (roundrect_rratio 0.25) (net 1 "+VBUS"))
  (pad "A5" smd roundrect (at -1.25 -3.68 270) (size 0.3 1.15) (layers "F.Cu" "F.Mask" "F.Paste") (roundrect_rratio 0.25) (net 11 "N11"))
  (pad "A6" smd roundrect (at -0.25 -3.68 270) (size 0.3 1.15) (layers "F.Cu" "F.Mask" "F.Paste") (roundrect_rratio 0.25)
   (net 8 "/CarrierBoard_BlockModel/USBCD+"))
  (pad "A7" smd roundrect (at 0.25 -3.68 270) (size 0.3 1.15) (layers "F.Cu" "F.Mask" "F.Paste") (roundrect_rratio 0.25)
   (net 7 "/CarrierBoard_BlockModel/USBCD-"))
  (pad "A8" smd roundrect (at 1.25 -3.68 270) (size 0.3 1.15) (layers "F.Cu" "F.Mask" "F.Paste") (roundrect_rratio 0.25) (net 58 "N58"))
  (pad "A9" smd roundrect (at 2.4 -3.68 270) (size 0.6 1.15) (layers "F.Cu" "F.Mask" "F.Paste") (roundrect_rratio 0.25) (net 1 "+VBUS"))
  (pad "A12" smd roundrect (at 3.2 -3.68 270) (size 0.6 1.15) (layers "F.Cu" "F.Mask" "F.Paste") (roundrect_rratio 0.25) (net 2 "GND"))
  (pad "B1" smd roundrect (at 3.2 -3.68 270) (size 0.6 1.15) (layers "F.Cu" "F.Mask" "F.Paste") (roundrect_rratio 0.25) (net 2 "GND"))
  (pad "B4" smd roundrect (at 2.4 -3.68 270) (size 0.6 1.15) (layers "F.Cu" "F.Mask" "F.Paste") (roundrect_rratio 0.25) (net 1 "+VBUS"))
  (pad "B5" smd roundrect (at 1.75 -3.68 270) (size 0.3 1.15) (layers "F.Cu" "F.Mask" "F.Paste") (roundrect_rratio 0.25) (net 4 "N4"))
  (pad "B6" smd roundrect (at 0.75 -3.68 270) (size 0.3 1.15) (layers "F.Cu" "F.Mask" "F.Paste") (roundrect_rratio 0.25)
   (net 8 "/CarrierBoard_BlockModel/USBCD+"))
  (pad "B7" smd roundrect (at -0.75 -3.68 270) (size 0.3 1.15) (layers "F.Cu" "F.Mask" "F.Paste") (roundrect_rratio 0.25)
   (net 7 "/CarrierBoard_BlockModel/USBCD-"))
  (pad "B8" smd roundrect (at -1.75 -3.68 270) (size 0.3 1.15) (layers "F.Cu" "F.Mask" "F.Paste") (roundrect_rratio 0.25) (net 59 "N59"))
  (pad "B9" smd roundrect (at -2.4 -3.68 270) (size 0.6 1.15) (layers "F.Cu" "F.Mask" "F.Paste") (roundrect_rratio 0.25) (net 1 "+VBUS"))
  (pad "B12" smd roundrect (at -3.2 -3.68 270) (size 0.6 1.15) (layers "F.Cu" "F.Mask" "F.Paste") (roundrect_rratio 0.25) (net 2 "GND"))
  (pad "S1" thru_hole oval (at -4.32 -3.105 270) (size 1 2.1) (drill oval 0.6 1.7) (layers "*.Cu" "*.Mask" "F.Paste")
   (remove_unused_layers no) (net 2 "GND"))
  (pad "S1" thru_hole oval (at -4.32 1.075 270) (size 1 1.8) (drill oval 0.6 1.4) (layers "*.Cu" "*.Mask" "F.Paste")
   (remove_unused_layers no) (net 2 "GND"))
  (pad "S1" thru_hole oval (at 4.32 -3.105 270) (size 1 2.1) (drill oval 0.6 1.7) (layers "*.Cu" "*.Mask" "F.Paste")
   (remove_unused_layers no) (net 2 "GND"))
  (pad "S1" thru_hole oval (at 4.32 1.075 270) (size 1 1.8) (drill oval 0.6 1.4) (layers "*.Cu" "*.Mask" "F.Paste")
   (remove_unused_layers no) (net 2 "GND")))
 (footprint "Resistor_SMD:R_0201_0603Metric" (layer "F.Cu") (at 104.980385 70.980385)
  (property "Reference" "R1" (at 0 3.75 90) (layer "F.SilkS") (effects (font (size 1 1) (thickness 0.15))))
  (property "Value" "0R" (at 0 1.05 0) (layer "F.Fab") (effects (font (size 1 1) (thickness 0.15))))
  (pad "" smd roundrect (at -0.345 0) (size 0.318 0.36) (layers "F.Paste") (roundrect_rratio 0.25))
  (pad "" smd roundrect (at 0.345 0) (size 0.318 0.36) (layers "F.Paste") (roundrect_rratio 0.25))
  (pad "1" smd roundrect (at -0.32 0) (size 0.46 0.4) (layers "F.Cu" "F.Mask") (roundrect_rratio 0.25) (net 1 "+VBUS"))
  (pad "2" smd roundrect (at 0.32 0) (size 0.46 0.4) (layers "F.Cu" "F.Mask") (roundrect_rratio 0.25) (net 3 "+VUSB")))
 (gr_rect (start 92.230385 45.230385) (end 168 90.230385) (stroke (width 0.05) (type default)) (fill no) (layer "Edge.Cuts"))
 (segment (start 99.410385 65.330385) (end 100.630385 65.330385) (width 0.5) (layer "F.Cu") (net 1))
 (segment (start 104.569385 71.030385) (end 104.619385 70.980385) (width 0.5) (layer "F.Cu") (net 1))
 (segment (start 100.630385 70.130385) (end 101.030385 70.130385) (width 0.5) (layer "F.Cu") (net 1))
 (segment (start 101.980385 71.080385) (end 102.830385 71.080385) (width 0.5) (layer "F.Cu") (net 1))
 (segment (start 99.410385 70.130385) (end 100.630385 70.130385) (width 0.5) (layer "F.Cu") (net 1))
 (segment (start 102.980385 71.030385) (end 104.569385 71.030385) (width 0.5) (layer "F.Cu") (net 1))
 (segment (start 101.030385 70.130385) (end 101.980385 71.080385) (width 0.5) (layer "F.Cu") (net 1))
 (via (at 100.630385 65.330385) (size 0.6) (drill 0.3) (layers "F.Cu" "B.Cu") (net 1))
 (via (at 100.630385 70.130385) (size 0.6) (drill 0.3) (layers "F.Cu" "B.Cu") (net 1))
 (via (at 105.842758 67.605386) (size 0.6) (drill 0.3) (layers "F.Cu" "B.Cu") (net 1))
 (segment (start 100.630385 65.330385) (end 100.630385 69.930385) (width 0.5) (layer "B.Cu") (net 1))
 (segment (start 99.410385 70.930385) (end 100.230385 70.930385) (width 0.5) (layer "F.Cu") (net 2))
 (segment (start 100.130385 64.530385) (end 100.330385 64.330385) (width 0.5) (layer "F.Cu") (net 2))
 (segment (start 100.630385 71.330385) (end 102.280385 72.980385) (width 0.5) (layer "F.Cu") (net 2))
 (segment (start 100.230385 70.930385) (end 100.630385 71.330385) (width 0.5) (layer "F.Cu") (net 2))
 (segment (start 102.980385 72.930385) (end 109.480385 72.930385) (width 0.5) (layer "F.Cu") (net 2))
 (segment (start 100.330385 64.330385) (end 100.530385 64.130385) (width 0.5) (layer "F.Cu") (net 2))
 (segment (start 100.530385 64.130385) (end 100.630385 64.030385) (width 0.5) (layer "F.Cu") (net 2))
 (segment (start 99.410385 64.530385) (end 100.130385 64.530385) (width 0.5) (layer "F.Cu") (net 2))
 (segment (start 102.280385 72.980385) (end 102.830385 72.980385) (width 0.5) (layer "F.Cu") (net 2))
 (via (at 100.630385 71.330385) (size 0.6) (drill 0.3) (layers "F.Cu" "B.Cu") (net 2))
 (via (at 100.630385 64.030385) (size 0.6) (drill 0.3) (layers "F.Cu" "B.Cu") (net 2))
 (segment (start 105.391385 71.030385) (end 105.341385 70.980385) (width 0.5) (layer "F.Cu") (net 3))
 (segment (start 115.730385 73.730385) (end 115.680385 73.680385) (width 0.25) (layer "F.Cu") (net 3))
 (segment (start 115.680385 73.680385) (end 115.680385 73.180385) (width 0.25) (layer "F.Cu") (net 3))
 (segment (start 113.530385 71.030385) (end 109.480385 71.030385) (width 0.25) (layer "F.Cu") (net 3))
 (segment (start 115.680385 73.180385) (end 113.530385 71.030385) (width 0.25) (layer "F.Cu") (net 3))
 (segment (start 107.230385 71.030385) (end 105.391385 71.030385) (width 0.5) (layer "F.Cu") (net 3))
 (segment (start 116.855385 73.180385) (end 115.680385 73.180385) (width 0.25) (layer "F.Cu") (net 3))
 (segment (start 115.780385 73.680385) (end 115.730385 73.730385) (width 0.25) (layer "F.Cu") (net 3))
 (segment (start 107.230385 71.030385) (end 109.480385 71.030385) (width 0.5) (layer "F.Cu") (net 3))
 (segment (start 116.855385 73.680385) (end 115.780385 73.680385) (width 0.25) (layer "F.Cu") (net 3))
 (segment (start 101.080385 66.980385) (end 101.280385 66.780385) (width 0.25) (layer "F.Cu") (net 7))
 (segment (start 101.080385 67.380385) (end 101.080385 66.980385) (width 0.25) (layer "F.Cu") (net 7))
 (segment (start 101.280385 66.780385) (end 104.192885 66.780385) (width 0.25) (layer "F.Cu") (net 7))
 (segment (start 99.410385 66.980385) (end 101.080385 66.980385) (width 0.25) (layer "F.Cu") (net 7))
 (segment (start 99.410385 67.980385) (end 100.480385 67.980385) (width 0.25) (layer "F.Cu") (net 7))
 (segment (start 100.480385 67.980385) (end 101.080385 67.380385) (width 0.25) (layer "F.Cu") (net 7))
 (segment (start 99.410385 68.480385) (end 101.780385 68.480385) (width 0.25) (layer "F.Cu") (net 8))
 (segment (start 98.430385 67.816207) (end 98.430385 68.144563) (width 0.25) (layer "F.Cu") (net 8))
 (segment (start 101.780385 68.480385) (end 101.980385 68.680385) (width 0.25) (layer "F.Cu") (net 8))
 (segment (start 98.766207 68.480385) (end 99.410385 68.480385) (width 0.25) (layer "F.Cu") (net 8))
 (segment (start 99.410385 67.480385) (end 98.766207 67.480385) (width 0.25) (layer "F.Cu") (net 8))
 (segment (start 98.766207 67.480385) (end 98.430385 67.816207) (width 0.25) (layer "F.Cu") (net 8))
 (segment (start 98.430385 68.144563) (end 98.766207 68.480385) (width 0.25) (layer "F.Cu") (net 8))
 (segment (start 101.980385 68.680385) (end 104.192885 68.680385) (width 0.25) (layer "F.Cu") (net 8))
 (segment (start 99.410385 69.480385) (end 100.780385 69.480385) (width 0.25) (layer "F.Cu") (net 4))
 (segment (start 100.780385 69.480385) (end 100.930385 69.330385) (width 0.25) (layer "F.Cu") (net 4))
 (segment (start 100.930385 69.330385) (end 101.555385 69.330385) (width 0.25) (layer "F.Cu") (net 4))
 (segment (start 100.830385 66.130385) (end 101.555385 66.130385) (width 0.25) (layer "F.Cu") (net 11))
 (segment (start 100.480385 66.480385) (end 100.830385 66.130385) (width 0.25) (layer "F.Cu") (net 11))
 (segment (start 99.410385 66.480385) (end 100.480385 66.480385) (width 0.25) (layer "F.Cu") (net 11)))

